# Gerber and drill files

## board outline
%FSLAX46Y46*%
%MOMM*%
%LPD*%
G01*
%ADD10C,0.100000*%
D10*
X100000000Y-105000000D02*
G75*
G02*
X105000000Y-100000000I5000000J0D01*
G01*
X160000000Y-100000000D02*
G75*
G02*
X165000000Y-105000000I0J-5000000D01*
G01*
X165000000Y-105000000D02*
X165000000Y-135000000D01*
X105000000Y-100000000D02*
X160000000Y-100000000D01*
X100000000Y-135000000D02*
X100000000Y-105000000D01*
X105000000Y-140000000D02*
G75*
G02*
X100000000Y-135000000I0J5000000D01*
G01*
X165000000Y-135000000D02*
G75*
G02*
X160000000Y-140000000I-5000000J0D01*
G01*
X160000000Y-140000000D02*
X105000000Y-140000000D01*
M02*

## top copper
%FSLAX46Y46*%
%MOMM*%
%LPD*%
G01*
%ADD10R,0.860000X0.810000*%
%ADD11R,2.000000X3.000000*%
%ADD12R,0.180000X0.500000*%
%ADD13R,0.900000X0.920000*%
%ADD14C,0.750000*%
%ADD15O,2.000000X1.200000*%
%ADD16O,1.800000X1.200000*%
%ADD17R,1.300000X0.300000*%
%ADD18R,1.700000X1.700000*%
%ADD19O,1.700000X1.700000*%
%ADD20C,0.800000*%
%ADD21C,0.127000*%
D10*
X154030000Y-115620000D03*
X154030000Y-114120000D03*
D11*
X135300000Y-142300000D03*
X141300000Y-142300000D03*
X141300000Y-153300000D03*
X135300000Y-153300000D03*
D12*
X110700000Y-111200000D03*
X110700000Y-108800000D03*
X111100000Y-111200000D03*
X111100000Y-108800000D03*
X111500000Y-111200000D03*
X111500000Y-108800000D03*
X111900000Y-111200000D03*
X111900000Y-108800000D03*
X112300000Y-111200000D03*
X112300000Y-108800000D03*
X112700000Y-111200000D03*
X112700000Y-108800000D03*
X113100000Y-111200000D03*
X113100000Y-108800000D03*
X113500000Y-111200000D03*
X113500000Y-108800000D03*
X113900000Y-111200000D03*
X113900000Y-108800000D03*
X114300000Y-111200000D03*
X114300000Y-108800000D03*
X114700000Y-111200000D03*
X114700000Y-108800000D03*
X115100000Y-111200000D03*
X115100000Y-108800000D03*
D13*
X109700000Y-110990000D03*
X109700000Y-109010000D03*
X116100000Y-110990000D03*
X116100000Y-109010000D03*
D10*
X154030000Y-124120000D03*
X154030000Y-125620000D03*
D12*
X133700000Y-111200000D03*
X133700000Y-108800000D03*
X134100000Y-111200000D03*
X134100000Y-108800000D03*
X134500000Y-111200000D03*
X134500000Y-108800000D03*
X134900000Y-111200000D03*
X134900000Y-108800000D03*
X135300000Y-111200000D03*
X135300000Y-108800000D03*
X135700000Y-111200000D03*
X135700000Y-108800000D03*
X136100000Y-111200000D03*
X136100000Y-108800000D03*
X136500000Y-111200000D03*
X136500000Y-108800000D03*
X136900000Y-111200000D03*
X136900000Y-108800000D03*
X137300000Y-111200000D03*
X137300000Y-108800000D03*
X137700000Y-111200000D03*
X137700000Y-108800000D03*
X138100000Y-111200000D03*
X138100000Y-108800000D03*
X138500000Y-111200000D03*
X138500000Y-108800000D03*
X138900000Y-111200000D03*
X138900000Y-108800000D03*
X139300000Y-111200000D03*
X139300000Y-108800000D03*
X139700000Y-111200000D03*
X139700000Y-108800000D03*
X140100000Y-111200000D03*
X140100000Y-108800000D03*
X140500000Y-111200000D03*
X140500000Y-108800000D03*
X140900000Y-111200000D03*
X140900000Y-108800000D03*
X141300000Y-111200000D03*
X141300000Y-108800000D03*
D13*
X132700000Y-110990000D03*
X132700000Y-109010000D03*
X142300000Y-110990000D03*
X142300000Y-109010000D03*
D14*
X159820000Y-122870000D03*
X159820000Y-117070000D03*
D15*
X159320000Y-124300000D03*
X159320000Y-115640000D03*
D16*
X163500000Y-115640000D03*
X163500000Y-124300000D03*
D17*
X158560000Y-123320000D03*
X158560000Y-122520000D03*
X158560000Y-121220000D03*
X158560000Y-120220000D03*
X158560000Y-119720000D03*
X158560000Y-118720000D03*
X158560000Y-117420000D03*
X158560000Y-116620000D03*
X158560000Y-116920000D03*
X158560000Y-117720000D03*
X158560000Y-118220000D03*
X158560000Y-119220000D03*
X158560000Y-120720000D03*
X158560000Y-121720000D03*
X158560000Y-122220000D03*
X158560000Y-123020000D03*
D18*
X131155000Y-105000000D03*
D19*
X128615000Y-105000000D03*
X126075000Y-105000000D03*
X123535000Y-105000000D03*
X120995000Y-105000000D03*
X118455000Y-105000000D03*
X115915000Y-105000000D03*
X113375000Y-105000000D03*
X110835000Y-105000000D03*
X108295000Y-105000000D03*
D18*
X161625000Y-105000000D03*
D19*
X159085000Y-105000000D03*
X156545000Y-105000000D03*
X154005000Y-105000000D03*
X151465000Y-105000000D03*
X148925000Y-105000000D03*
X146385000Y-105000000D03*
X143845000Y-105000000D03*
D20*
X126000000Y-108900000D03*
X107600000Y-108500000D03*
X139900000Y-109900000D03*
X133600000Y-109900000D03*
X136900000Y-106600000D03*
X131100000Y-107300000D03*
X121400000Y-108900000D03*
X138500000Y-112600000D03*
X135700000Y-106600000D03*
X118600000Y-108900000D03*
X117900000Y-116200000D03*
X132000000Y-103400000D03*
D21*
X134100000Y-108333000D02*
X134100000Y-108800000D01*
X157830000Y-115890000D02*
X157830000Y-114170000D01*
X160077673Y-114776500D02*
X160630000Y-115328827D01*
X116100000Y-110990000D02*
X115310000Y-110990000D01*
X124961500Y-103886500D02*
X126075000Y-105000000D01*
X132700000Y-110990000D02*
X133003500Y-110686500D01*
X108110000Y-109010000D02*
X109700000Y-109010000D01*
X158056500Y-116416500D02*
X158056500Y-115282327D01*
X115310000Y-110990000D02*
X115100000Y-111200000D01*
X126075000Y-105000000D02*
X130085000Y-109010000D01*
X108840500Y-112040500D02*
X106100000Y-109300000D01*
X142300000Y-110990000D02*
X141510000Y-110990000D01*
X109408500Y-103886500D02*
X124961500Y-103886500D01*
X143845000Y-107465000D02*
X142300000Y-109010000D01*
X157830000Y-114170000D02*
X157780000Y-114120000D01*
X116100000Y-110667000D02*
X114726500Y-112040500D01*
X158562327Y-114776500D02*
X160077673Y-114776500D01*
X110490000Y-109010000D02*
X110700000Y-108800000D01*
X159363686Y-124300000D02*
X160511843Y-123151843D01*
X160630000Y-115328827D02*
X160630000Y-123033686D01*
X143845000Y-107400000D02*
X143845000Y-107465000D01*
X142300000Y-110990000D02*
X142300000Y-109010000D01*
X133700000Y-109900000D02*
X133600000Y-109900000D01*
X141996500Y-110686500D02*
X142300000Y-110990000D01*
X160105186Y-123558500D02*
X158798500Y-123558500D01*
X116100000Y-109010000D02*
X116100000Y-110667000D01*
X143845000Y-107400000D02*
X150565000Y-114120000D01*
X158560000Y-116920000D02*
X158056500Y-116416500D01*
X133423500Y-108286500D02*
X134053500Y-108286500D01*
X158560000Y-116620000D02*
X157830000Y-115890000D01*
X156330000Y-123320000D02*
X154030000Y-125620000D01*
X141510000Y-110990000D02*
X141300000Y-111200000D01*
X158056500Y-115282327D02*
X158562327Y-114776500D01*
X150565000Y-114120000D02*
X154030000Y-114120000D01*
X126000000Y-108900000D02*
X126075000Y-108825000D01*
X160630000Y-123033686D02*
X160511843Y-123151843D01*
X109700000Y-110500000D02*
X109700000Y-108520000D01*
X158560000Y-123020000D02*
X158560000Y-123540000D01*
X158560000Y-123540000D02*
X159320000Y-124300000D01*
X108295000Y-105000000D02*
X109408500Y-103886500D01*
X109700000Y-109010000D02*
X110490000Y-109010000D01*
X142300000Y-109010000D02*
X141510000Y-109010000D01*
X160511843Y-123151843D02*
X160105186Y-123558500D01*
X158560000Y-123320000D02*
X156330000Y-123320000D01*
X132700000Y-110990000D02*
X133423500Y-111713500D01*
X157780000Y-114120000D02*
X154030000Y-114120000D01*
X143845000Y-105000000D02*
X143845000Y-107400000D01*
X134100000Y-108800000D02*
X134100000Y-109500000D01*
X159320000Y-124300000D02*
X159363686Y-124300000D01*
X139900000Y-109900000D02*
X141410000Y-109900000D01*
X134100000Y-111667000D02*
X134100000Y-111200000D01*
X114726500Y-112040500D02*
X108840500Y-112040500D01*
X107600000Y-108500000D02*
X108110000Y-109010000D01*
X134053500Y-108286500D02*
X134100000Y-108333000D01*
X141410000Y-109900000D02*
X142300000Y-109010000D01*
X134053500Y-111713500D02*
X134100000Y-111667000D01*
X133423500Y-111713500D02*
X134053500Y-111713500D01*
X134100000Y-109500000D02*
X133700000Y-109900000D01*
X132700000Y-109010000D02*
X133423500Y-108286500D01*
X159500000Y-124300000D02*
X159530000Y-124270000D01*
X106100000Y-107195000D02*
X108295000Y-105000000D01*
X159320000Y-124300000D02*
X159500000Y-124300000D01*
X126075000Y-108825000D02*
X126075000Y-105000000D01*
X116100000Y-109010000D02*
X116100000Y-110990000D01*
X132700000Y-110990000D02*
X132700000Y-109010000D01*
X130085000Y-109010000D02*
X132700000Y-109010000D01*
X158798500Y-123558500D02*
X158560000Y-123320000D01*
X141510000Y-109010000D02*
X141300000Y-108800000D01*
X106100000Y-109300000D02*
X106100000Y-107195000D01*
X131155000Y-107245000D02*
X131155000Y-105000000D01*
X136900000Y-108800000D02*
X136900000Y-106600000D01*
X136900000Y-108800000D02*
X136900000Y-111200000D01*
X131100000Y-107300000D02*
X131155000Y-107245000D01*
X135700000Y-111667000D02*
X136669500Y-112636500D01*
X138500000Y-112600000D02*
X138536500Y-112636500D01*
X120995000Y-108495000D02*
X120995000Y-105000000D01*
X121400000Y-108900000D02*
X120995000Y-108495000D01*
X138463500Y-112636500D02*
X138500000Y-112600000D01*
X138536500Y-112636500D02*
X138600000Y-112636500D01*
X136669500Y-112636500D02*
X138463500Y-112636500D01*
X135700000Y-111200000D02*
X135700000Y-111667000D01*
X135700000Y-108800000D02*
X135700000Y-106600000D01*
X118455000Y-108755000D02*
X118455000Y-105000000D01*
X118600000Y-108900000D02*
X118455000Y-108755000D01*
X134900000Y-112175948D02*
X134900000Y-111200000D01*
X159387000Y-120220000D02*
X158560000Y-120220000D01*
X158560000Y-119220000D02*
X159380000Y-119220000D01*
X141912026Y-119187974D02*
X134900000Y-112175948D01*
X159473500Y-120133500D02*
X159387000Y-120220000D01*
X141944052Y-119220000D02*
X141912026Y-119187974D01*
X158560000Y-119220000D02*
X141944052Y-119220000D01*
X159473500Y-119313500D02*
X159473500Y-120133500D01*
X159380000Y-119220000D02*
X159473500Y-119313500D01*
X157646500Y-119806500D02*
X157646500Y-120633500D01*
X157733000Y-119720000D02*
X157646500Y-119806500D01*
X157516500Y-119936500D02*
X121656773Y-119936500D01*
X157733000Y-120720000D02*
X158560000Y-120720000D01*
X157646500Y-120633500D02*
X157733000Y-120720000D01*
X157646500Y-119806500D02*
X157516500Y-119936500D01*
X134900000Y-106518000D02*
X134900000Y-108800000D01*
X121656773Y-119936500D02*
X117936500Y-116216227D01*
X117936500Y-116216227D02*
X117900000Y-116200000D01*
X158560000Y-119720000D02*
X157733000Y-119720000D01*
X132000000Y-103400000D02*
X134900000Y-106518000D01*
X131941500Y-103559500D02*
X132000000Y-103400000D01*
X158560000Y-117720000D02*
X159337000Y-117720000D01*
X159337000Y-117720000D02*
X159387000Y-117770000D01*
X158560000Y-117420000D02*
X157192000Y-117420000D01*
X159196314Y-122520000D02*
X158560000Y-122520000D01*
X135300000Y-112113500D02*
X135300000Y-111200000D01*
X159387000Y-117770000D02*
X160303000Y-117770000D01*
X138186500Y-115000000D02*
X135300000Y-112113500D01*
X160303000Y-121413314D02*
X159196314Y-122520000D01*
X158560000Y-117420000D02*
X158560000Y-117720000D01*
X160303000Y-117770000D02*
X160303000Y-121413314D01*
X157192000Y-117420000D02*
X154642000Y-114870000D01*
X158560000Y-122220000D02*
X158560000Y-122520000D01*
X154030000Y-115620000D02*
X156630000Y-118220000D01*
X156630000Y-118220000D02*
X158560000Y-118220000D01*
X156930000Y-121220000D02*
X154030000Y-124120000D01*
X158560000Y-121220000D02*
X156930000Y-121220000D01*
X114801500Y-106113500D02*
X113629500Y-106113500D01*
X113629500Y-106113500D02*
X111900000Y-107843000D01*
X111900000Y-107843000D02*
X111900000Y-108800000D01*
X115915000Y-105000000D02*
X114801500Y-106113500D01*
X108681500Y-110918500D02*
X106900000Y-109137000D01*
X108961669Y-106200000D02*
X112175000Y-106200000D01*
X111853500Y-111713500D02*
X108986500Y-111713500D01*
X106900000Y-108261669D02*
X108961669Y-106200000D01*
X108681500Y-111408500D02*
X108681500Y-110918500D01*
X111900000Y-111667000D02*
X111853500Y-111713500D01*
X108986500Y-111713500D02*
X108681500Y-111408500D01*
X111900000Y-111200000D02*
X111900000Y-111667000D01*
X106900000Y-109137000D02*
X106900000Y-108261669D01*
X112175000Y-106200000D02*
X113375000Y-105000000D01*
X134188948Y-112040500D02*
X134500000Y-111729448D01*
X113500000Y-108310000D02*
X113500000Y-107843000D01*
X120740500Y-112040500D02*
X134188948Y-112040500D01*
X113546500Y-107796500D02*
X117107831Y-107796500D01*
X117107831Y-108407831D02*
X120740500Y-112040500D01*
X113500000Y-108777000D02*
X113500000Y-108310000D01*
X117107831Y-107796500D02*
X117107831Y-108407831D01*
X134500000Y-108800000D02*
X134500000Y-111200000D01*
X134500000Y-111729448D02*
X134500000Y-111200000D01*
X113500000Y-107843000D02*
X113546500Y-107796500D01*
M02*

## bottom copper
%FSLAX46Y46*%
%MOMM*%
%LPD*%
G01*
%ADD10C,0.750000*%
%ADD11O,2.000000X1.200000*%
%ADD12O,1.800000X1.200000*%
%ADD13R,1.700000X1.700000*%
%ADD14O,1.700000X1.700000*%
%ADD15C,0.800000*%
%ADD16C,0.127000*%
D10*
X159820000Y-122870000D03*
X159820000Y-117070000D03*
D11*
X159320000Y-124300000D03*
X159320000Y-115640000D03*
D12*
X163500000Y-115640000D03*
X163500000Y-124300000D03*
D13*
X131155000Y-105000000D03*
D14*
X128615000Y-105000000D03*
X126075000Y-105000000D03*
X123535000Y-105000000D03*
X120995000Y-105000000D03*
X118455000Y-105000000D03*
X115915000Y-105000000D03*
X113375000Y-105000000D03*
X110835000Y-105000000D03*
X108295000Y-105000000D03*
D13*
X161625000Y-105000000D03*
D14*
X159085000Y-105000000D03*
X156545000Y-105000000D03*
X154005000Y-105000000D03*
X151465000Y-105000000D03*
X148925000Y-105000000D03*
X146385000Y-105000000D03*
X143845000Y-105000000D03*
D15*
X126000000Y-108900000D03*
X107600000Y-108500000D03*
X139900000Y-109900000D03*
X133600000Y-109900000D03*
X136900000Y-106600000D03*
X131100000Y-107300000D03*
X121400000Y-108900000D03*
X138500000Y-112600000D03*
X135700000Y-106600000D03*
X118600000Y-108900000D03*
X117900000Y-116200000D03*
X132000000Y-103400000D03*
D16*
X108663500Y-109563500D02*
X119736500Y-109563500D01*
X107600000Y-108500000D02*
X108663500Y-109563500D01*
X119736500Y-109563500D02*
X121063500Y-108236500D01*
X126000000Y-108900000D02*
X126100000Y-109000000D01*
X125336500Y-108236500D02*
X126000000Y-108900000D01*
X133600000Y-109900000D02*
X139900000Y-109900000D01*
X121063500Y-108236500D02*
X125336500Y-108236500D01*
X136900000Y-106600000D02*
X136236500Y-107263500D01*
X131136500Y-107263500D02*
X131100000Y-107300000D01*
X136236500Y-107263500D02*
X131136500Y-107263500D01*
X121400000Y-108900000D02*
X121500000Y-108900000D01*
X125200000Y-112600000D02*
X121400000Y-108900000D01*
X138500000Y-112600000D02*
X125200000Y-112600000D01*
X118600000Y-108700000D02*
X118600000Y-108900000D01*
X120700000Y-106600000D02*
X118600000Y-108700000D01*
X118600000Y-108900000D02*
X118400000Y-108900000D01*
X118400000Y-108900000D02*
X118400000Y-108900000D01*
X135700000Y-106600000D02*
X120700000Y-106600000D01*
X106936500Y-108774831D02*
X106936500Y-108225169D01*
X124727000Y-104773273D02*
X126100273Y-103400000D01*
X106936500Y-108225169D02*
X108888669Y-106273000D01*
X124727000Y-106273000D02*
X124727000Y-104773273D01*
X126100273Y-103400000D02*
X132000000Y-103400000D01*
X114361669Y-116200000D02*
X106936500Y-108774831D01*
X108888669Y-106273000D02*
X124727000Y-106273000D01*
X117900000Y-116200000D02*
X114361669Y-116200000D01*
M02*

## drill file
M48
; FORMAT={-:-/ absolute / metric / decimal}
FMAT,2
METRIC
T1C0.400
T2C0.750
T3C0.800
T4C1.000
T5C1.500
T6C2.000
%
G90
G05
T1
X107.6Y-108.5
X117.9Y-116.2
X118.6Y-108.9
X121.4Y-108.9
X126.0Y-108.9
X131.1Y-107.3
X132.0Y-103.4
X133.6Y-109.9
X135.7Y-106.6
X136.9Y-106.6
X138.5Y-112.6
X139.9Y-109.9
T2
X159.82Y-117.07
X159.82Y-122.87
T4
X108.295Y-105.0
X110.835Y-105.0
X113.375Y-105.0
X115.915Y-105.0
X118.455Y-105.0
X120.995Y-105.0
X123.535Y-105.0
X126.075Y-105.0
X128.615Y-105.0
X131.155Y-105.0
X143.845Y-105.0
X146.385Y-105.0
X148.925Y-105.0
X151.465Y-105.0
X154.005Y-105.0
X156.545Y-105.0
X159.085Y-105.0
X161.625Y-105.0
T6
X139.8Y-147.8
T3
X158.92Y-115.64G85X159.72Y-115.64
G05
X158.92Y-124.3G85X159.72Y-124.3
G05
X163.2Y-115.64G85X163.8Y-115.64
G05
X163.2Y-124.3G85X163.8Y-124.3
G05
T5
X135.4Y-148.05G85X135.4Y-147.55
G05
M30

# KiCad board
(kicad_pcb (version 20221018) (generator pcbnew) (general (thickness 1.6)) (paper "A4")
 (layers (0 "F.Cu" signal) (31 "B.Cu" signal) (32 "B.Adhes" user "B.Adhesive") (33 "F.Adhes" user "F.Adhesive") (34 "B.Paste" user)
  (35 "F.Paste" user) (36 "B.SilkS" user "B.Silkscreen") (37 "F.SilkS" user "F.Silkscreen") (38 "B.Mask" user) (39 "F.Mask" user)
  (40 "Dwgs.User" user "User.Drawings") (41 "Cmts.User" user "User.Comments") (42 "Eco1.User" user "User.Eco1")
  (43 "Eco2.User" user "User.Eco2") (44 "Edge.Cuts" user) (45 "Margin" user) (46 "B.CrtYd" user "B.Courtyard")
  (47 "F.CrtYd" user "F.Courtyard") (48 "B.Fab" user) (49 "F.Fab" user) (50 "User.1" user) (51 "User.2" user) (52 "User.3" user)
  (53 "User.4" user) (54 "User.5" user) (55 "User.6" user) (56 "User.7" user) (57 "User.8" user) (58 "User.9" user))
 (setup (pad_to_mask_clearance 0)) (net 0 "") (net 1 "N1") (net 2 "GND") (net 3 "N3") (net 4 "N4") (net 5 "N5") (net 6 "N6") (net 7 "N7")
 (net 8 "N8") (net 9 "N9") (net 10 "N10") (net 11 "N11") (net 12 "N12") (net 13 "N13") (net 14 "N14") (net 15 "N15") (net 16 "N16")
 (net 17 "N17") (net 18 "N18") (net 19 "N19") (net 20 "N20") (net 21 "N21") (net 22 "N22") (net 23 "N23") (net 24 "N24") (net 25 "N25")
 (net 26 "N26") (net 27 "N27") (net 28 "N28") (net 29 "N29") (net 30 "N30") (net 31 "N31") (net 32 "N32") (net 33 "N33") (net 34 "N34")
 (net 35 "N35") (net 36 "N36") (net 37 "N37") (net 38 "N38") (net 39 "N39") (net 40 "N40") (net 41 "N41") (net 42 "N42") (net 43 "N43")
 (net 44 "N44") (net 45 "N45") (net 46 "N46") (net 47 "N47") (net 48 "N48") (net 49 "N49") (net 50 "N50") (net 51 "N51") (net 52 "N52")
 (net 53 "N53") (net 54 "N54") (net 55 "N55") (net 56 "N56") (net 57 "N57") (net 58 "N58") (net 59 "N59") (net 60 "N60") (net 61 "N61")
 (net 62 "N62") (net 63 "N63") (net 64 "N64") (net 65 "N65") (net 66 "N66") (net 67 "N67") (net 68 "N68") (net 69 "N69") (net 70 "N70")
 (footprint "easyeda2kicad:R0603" (layer "F.Cu") (at 154.03 114.87 90)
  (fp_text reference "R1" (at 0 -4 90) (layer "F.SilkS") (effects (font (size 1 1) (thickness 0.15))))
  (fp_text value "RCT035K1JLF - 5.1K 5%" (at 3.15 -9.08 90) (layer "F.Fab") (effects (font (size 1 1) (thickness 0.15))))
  (pad "1" smd rect (at -0.75 0 90) (size 0.81 0.86) (layers "F.Cu" "F.Paste" "F.Mask") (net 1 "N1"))
  (pad "2" smd rect (at 0.75 0 90) (size 0.81 0.86) (layers "F.Cu" "F.Paste" "F.Mask") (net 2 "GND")))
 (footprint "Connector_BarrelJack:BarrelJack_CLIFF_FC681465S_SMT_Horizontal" (layer "F.Cu") (at 138.3 147.8)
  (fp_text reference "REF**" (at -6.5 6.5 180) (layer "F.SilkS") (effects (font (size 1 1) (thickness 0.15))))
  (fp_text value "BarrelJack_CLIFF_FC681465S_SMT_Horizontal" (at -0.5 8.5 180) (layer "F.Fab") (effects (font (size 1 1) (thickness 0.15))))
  (pad "" np_thru_hole oval (at -2.9 0 90) (size 2 1.5) (drill oval 2 1.5) (layers "*.Cu" "*.Mask"))
  (pad "" np_thru_hole circle (at 1.5 0 90) (size 2 2) (drill 2) (layers "*.Cu" "*.Mask"))
  (pad "1" smd rect (at -3 -5.5 90) (size 3 2) (layers "F.Cu" "F.Paste" "F.Mask"))
  (pad "1" smd rect (at 3 -5.5 90) (size 3 2) (layers "F.Cu" "F.Paste" "F.Mask"))
  (pad "2" smd rect (at 3 5.5 90) (size 3 2) (layers "F.Cu" "F.Paste" "F.Mask"))
  (pad "3" smd rect (at -3 5.5 90) (size 3 2) (layers "F.Cu" "F.Paste" "F.Mask")))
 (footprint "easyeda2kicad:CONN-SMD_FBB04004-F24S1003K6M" (layer "F.Cu") (at 112.9 110)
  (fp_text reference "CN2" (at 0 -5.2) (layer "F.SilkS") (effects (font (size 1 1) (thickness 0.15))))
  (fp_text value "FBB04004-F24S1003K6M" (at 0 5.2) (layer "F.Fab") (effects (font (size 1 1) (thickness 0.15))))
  (pad "1" smd rect (at -2.2 1.2) (size 0.18 0.5) (layers "F.Cu" "F.Paste" "F.Mask") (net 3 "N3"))
  (pad "2" smd rect (at -2.2 -1.2) (size 0.18 0.5) (layers "F.Cu" "F.Paste" "F.Mask") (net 2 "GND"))
  (pad "3" smd rect (at -1.8 1.2) (size 0.18 0.5) (layers "F.Cu" "F.Paste" "F.Mask") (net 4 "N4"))
  (pad "4" smd rect (at -1.8 -1.2) (size 0.18 0.5) (layers "F.Cu" "F.Paste" "F.Mask") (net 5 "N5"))
  (pad "5" smd rect (at -1.4 1.2) (size 0.18 0.5) (layers "F.Cu" "F.Paste" "F.Mask") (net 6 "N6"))
  (pad "6" smd rect (at -1.4 -1.2) (size 0.18 0.5) (layers "F.Cu" "F.Paste" "F.Mask") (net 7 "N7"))
  (pad "7" smd rect (at -1 1.2) (size 0.18 0.5) (layers "F.Cu" "F.Paste" "F.Mask") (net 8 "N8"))
  (pad "8" smd rect (at -1 -1.2) (size 0.18 0.5) (layers "F.Cu" "F.Paste" "F.Mask") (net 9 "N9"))
  (pad "9" smd rect (at -0.6 1.2) (size 0.18 0.5) (layers "F.Cu" "F.Paste" "F.Mask") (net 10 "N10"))
  (pad "10" smd rect (at -0.6 -1.2) (size 0.18 0.5) (layers "F.Cu" "F.Paste" "F.Mask") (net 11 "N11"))
  (pad "11" smd rect (at -0.2 1.2) (size 0.18 0.5) (layers "F.Cu" "F.Paste" "F.Mask") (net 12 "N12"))
  (pad "12" smd rect (at -0.2 -1.2) (size 0.18 0.5) (layers "F.Cu" "F.Paste" "F.Mask") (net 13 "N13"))
  (pad "13" smd rect (at 0.2 1.2) (size 0.18 0.5) (layers "F.Cu" "F.Paste" "F.Mask") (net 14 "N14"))
  (pad "14" smd rect (at 0.2 -1.2) (size 0.18 0.5) (layers "F.Cu" "F.Paste" "F.Mask") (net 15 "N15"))
  (pad "15" smd rect (at 0.6 1.2) (size 0.18 0.5) (layers "F.Cu" "F.Paste" "F.Mask") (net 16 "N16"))
  (pad "16" smd rect (at 0.6 -1.2) (size 0.18 0.5) (layers "F.Cu" "F.Paste" "F.Mask") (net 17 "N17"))
  (pad "17" smd rect (at 1 1.2) (size 0.18 0.5) (layers "F.Cu" "F.Paste" "F.Mask") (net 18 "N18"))
  (pad "18" smd rect (at 1 -1.2) (size 0.18 0.5) (layers "F.Cu" "F.Paste" "F.Mask") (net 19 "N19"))
  (pad "19" smd rect (at 1.4 1.2) (size 0.18 0.5) (layers "F.Cu" "F.Paste" "F.Mask") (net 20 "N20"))
  (pad "20" smd rect (at 1.4 -1.2) (size 0.18 0.5) (layers "F.Cu" "F.Paste" "F.Mask") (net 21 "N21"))
  (pad "21" smd rect (at 1.8 1.2) (size 0.18 0.5) (layers "F.Cu" "F.Paste" "F.Mask") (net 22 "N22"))
  (pad "22" smd rect (at 1.8 -1.2) (size 0.18 0.5) (layers "F.Cu" "F.Paste" "F.Mask") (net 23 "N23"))
  (pad "23" smd rect (at 2.2 1.2) (size 0.18 0.5) (layers "F.Cu" "F.Paste" "F.Mask") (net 2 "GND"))
  (pad "24" smd rect (at 2.2 -1.2) (size 0.18 0.5) (layers "F.Cu" "F.Paste" "F.Mask") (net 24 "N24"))
  (pad "25" smd rect (at -3.2 0.99) (size 0.9 0.92) (layers "F.Cu" "F.Paste" "F.Mask") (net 2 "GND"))
  (pad "26" smd rect (at -3.2 -0.99) (size 0.9 0.92) (layers "F.Cu" "F.Paste" "F.Mask") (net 2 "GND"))
  (pad "27" smd rect (at 3.2 0.99) (size 0.9 0.92) (layers "F.Cu" "F.Paste" "F.Mask") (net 2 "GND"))
  (pad "28" smd rect (at 3.2 -0.99) (size 0.9 0.92) (layers "F.Cu" "F.Paste" "F.Mask") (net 2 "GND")))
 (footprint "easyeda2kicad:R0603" (layer "F.Cu") (at 154.03 124.87 -90)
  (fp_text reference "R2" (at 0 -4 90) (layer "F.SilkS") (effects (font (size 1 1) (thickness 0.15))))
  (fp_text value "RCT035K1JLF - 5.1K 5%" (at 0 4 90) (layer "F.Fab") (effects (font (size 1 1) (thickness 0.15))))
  (pad "1" smd rect (at -0.75 0 270) (size 0.81 0.86) (layers "F.Cu" "F.Paste" "F.Mask") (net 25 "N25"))
  (pad "2" smd rect (at 0.75 0 270) (size 0.81 0.86) (layers "F.Cu" "F.Paste" "F.Mask") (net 2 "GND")))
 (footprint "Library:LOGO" (layer "F.Cu") (at 156.4 132.7)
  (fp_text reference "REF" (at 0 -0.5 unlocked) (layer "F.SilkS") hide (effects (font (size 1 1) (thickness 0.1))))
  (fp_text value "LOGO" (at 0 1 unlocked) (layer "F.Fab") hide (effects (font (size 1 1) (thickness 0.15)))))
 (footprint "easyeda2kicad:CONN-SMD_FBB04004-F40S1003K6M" (layer "F.Cu") (at 137.5 110)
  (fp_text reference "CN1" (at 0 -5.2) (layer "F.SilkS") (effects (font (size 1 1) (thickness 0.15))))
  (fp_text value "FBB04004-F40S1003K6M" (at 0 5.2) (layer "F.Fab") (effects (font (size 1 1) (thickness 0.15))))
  (pad "1" smd rect (at -3.8 1.2) (size 0.18 0.5) (layers "F.Cu" "F.Paste" "F.Mask") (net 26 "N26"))
  (pad "2" smd rect (at -3.8 -1.2) (size 0.18 0.5) (layers "F.Cu" "F.Paste" "F.Mask") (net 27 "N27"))
  (pad "3" smd rect (at -3.4 1.2) (size 0.18 0.5) (layers "F.Cu" "F.Paste" "F.Mask") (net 2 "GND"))
  (pad "4" smd rect (at -3.4 -1.2) (size 0.18 0.5) (layers "F.Cu" "F.Paste" "F.Mask") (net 2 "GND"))
  (pad "5" smd rect (at -3 1.2) (size 0.18 0.5) (layers "F.Cu" "F.Paste" "F.Mask") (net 17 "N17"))
  (pad "6" smd rect (at -3 -1.2) (size 0.18 0.5) (layers "F.Cu" "F.Paste" "F.Mask") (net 17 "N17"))
  (pad "7" smd rect (at -2.6 1.2) (size 0.18 0.5) (layers "F.Cu" "F.Paste" "F.Mask") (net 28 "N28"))
  (pad "8" smd rect (at -2.6 -1.2) (size 0.18 0.5) (layers "F.Cu" "F.Paste" "F.Mask") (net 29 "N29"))
  (pad "9" smd rect (at -2.2 1.2) (size 0.18 0.5) (layers "F.Cu" "F.Paste" "F.Mask") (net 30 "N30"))
  (pad "10" smd rect (at -2.2 -1.2) (size 0.18 0.5) (layers "F.Cu" "F.Paste" "F.Mask") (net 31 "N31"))
  (pad "11" smd rect (at -1.8 1.2) (size 0.18 0.5) (layers "F.Cu" "F.Paste" "F.Mask") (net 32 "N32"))
  (pad "12" smd rect (at -1.8 -1.2) (size 0.18 0.5) (layers "F.Cu" "F.Paste" "F.Mask") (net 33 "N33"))
  (pad "13" smd rect (at -1.4 1.2) (size 0.18 0.5) (layers "F.Cu" "F.Paste" "F.Mask") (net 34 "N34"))
  (pad "14" smd rect (at -1.4 -1.2) (size 0.18 0.5) (layers "F.Cu" "F.Paste" "F.Mask") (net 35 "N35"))
  (pad "15" smd rect (at -1 1.2) (size 0.18 0.5) (layers "F.Cu" "F.Paste" "F.Mask") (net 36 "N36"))
  (pad "16" smd rect (at -1 -1.2) (size 0.18 0.5) (layers "F.Cu" "F.Paste" "F.Mask") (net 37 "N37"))
  (pad "17" smd rect (at -0.6 1.2) (size 0.18 0.5) (layers "F.Cu" "F.Paste" "F.Mask") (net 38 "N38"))
  (pad "18" smd rect (at -0.6 -1.2) (size 0.18 0.5) (layers "F.Cu" "F.Paste" "F.Mask") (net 38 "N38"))
  (pad "19" smd rect (at -0.2 1.2) (size 0.18 0.5) (layers "F.Cu" "F.Paste" "F.Mask") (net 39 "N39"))
  (pad "20" smd rect (at -0.2 -1.2) (size 0.18 0.5) (layers "F.Cu" "F.Paste" "F.Mask") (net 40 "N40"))
  (pad "21" smd rect (at 0.2 1.2) (size 0.18 0.5) (layers "F.Cu" "F.Paste" "F.Mask") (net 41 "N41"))
  (pad "22" smd rect (at 0.2 -1.2) (size 0.18 0.5) (layers "F.Cu" "F.Paste" "F.Mask") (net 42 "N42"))
  (pad "23" smd rect (at 0.6 1.2) (size 0.18 0.5) (layers "F.Cu" "F.Paste" "F.Mask") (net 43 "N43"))
  (pad "24" smd rect (at 0.6 -1.2) (size 0.18 0.5) (layers "F.Cu" "F.Paste" "F.Mask") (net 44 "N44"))
  (pad "25" smd rect (at 1 1.2) (size 0.18 0.5) (layers "F.Cu" "F.Paste" "F.Mask") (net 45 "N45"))
  (pad "26" smd rect (at 1 -1.2) (size 0.18 0.5) (layers "F.Cu" "F.Paste" "F.Mask") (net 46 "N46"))
  (pad "27" smd rect (at 1.4 1.2) (size 0.18 0.5) (layers "F.Cu" "F.Paste" "F.Mask") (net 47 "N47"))
  (pad "28" smd rect (at 1.4 -1.2) (size 0.18 0.5) (layers "F.Cu" "F.Paste" "F.Mask") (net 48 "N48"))
  (pad "29" smd rect (at 1.8 1.2) (size 0.18 0.5) (layers "F.Cu" "F.Paste" "F.Mask") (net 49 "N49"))
  (pad "30" smd rect (at 1.8 -1.2) (size 0.18 0.5) (layers "F.Cu" "F.Paste" "F.Mask") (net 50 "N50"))
  (pad "31" smd rect (at 2.2 1.2) (size 0.18 0.5) (layers "F.Cu" "F.Paste" "F.Mask") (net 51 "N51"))
  (pad "32" smd rect (at 2.2 -1.2) (size 0.18 0.5) (layers "F.Cu" "F.Paste" "F.Mask") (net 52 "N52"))
  (pad "33" smd rect (at 2.6 1.2) (size 0.18 0.5) (layers "F.Cu" "F.Paste" "F.Mask") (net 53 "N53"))
  (pad "34" smd rect (at 2.6 -1.2) (size 0.18 0.5) (layers "F.Cu" "F.Paste" "F.Mask") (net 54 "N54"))
  (pad "35" smd rect (at 3 1.2) (size 0.18 0.5) (layers "F.Cu" "F.Paste" "F.Mask") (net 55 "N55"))
  (pad "36" smd rect (at 3 -1.2) (size 0.18 0.5) (layers "F.Cu" "F.Paste" "F.Mask") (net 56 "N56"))
  (pad "37" smd rect (at 3.4 1.2) (size 0.18 0.5) (layers "F.Cu" "F.Paste" "F.Mask") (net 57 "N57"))
  (pad "38" smd rect (at 3.4 -1.2) (size 0.18 0.5) (layers "F.Cu" "F.Paste" "F.Mask") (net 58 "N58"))
  (pad "39" smd rect (at 3.8 1.2) (size 0.18 0.5) (layers "F.Cu" "F.Paste" "F.Mask") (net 2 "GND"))
  (pad "40" smd rect (at 3.8 -1.2) (size 0.18 0.5) (layers "F.Cu" "F.Paste" "F.Mask") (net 2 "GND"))
  (pad "41" smd rect (at -4.8 0.99) (size 0.9 0.92) (layers "F.Cu" "F.Paste" "F.Mask") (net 2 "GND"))
  (pad "42" smd rect (at -4.8 -0.99) (size 0.9 0.92) (layers "F.Cu" "F.Paste" "F.Mask") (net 2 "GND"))
  (pad "43" smd rect (at 4.8 0.99) (size 0.9 0.92) (layers "F.Cu" "F.Paste" "F.Mask") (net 2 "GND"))
  (pad "44" smd rect (at 4.8 -0.99) (size 0.9 0.92) (layers "F.Cu" "F.Paste" "F.Mask") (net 2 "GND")))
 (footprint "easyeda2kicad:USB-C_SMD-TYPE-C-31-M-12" (layer "F.Cu") (at 161.03 119.97 90)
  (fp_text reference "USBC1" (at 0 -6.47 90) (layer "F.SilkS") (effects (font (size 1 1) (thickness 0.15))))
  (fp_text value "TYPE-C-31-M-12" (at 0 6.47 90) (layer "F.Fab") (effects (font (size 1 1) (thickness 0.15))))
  (pad "" thru_hole circle (at -2.9 -1.21 90) (size 0.75 0.75) (drill 0.75) (layers "*.Cu" "*.Mask"))
  (pad "" thru_hole circle (at 2.9 -1.21 90) (size 0.75 0.75) (drill 0.75) (layers "*.Cu" "*.Mask"))
  (pad "0" thru_hole oval (at -4.33 -1.71 90) (size 1.2 2) (drill oval 0.799998 1.600022) (layers "*.Cu" "*.Mask") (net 2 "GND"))
  (pad "1" thru_hole oval (at 4.33 -1.71 90) (size 1.2 2) (drill oval 0.799998 1.599971) (layers "*.Cu" "*.Mask"))
  (pad "2" thru_hole oval (at 4.33 2.47 90) (size 1.2 1.8) (drill oval 0.799998 1.399997) (layers "*.Cu" "*.Mask"))
  (pad "3" thru_hole oval (at -4.33 2.47 90) (size 1.2 1.8) (drill oval 0.799998 1.399997) (layers "*.Cu" "*.Mask"))
  (pad "A1" smd rect (at -3.35 -2.47 90) (size 0.3 1.3) (layers "F.Cu" "F.Paste" "F.Mask") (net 2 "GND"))
  (pad "A4" smd rect (at -2.55 -2.47 90) (size 0.3 1.3) (layers "F.Cu" "F.Paste" "F.Mask") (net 30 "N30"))
  (pad "A5" smd rect (at -1.25 -2.47 90) (size 0.3 1.3) (layers "F.Cu" "F.Paste" "F.Mask") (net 25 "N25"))
  (pad "A6" smd rect (at -0.25 -2.47 90) (size 0.3 1.3) (layers "F.Cu" "F.Paste" "F.Mask") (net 28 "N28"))
  (pad "A7" smd rect (at 0.25 -2.47 90) (size 0.3 1.3) (layers "F.Cu" "F.Paste" "F.Mask") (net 29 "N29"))
  (pad "A8" smd rect (at 1.25 -2.47 90) (size 0.3 1.3) (layers "F.Cu" "F.Paste" "F.Mask") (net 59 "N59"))
  (pad "A9" smd rect (at 2.55 -2.47 90) (size 0.3 1.3) (layers "F.Cu" "F.Paste" "F.Mask") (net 30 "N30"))
  (pad "A12" smd rect (at 3.35 -2.47 90) (size 0.3 1.3) (layers "F.Cu" "F.Paste" "F.Mask") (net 2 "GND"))
  (pad "B1" smd rect (at 3.05 -2.47 90) (size 0.3 1.3) (layers "F.Cu" "F.Paste" "F.Mask") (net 2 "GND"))
  (pad "B4" smd rect (at 2.25 -2.47 90) (size 0.3 1.3) (layers "F.Cu" "F.Paste" "F.Mask") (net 30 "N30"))
  (pad "B5" smd rect (at 1.75 -2.47 90) (size 0.3 1.3) (layers "F.Cu" "F.Paste" "F.Mask") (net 1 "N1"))
  (pad "B6" smd rect (at 0.75 -2.47 90) (size 0.3 1.3) (layers "F.Cu" "F.Paste" "F.Mask") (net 28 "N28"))
  (pad "B7" smd rect (at -0.75 -2.47 90) (size 0.3 1.3) (layers "F.Cu" "F.Paste" "F.Mask") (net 29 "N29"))
  (pad "B8" smd rect (at -1.75 -2.47 90) (size 0.3 1.3) (layers "F.Cu" "F.Paste" "F.Mask") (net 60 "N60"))
  (pad "B9" smd rect (at -2.25 -2.47 90) (size 0.3 1.3) (layers "F.Cu" "F.Paste" "F.Mask") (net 30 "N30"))
  (pad "B12" smd rect (at -3.05 -2.47 90) (size 0.3 1.3) (layers "F.Cu" "F.Paste" "F.Mask") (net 2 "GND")))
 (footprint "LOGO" (layer "B.Cu") (at 156.4 132.7 180)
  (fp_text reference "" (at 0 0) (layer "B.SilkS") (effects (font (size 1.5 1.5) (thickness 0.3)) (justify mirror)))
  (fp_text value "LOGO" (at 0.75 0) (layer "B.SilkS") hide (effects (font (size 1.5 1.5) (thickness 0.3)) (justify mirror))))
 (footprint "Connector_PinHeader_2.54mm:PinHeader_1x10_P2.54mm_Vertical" (layer "B.Cu") (at 131.155 105 90)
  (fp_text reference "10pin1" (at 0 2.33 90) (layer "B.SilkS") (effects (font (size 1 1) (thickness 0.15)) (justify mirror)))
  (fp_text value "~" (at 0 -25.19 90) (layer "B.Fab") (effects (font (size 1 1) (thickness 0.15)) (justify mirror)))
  (pad "1" thru_hole rect (at 0 0 90) (size 1.7 1.7) (drill 1) (layers "*.Cu" "*.Mask") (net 38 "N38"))
  (pad "2" thru_hole oval (at 0 -2.54 90) (size 1.7 1.7) (drill 1) (layers "*.Cu" "*.Mask") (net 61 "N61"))
  (pad "3" thru_hole oval (at 0 -5.08 90) (size 1.7 1.7) (drill 1) (layers "*.Cu" "*.Mask") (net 2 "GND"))
  (pad "4" thru_hole oval (at 0 -7.62 90) (size 1.7 1.7) (drill 1) (layers "*.Cu" "*.Mask") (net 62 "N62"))
  (pad "5" thru_hole oval (at 0 -10.16 90) (size 1.7 1.7) (drill 1) (layers "*.Cu" "*.Mask") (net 32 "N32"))
  (pad "6" thru_hole oval (at 0 -12.7 90) (size 1.7 1.7) (drill 1) (layers "*.Cu" "*.Mask") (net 33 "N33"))
  (pad "7" thru_hole oval (at 0 -15.24 90) (size 1.7 1.7) (drill 1) (layers "*.Cu" "*.Mask") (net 9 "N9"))
  (pad "8" thru_hole oval (at 0 -17.78 90) (size 1.7 1.7) (drill 1) (layers "*.Cu" "*.Mask") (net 8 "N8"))
  (pad "9" thru_hole oval (at 0 -20.32 90) (size 1.7 1.7) (drill 1) (layers "*.Cu" "*.Mask") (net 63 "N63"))
  (pad "10" thru_hole oval (at 0 -22.86 90) (size 1.7 1.7) (drill 1) (layers "*.Cu" "*.Mask") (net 2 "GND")))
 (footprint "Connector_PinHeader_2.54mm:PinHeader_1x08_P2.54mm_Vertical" (layer "B.Cu") (at 161.625 105 90)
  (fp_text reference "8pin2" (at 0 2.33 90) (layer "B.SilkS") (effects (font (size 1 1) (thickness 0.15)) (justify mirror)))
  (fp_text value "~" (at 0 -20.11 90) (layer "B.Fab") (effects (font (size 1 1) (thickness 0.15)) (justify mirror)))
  (pad "1" thru_hole rect (at 0 0 90) (size 1.7 1.7) (drill 1) (layers "*.Cu" "*.Mask") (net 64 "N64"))
  (pad "2" thru_hole oval (at 0 -2.54 90) (size 1.7 1.7) (drill 1) (layers "*.Cu" "*.Mask") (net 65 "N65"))
  (pad "3" thru_hole oval (at 0 -5.08 90) (size 1.7 1.7) (drill 1) (layers "*.Cu" "*.Mask") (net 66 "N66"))
  (pad "4" thru_hole oval (at 0 -7.62 90) (size 1.7 1.7) (drill 1) (layers "*.Cu" "*.Mask") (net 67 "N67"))
  (pad "5" thru_hole oval (at 0 -10.16 90) (size 1.7 1.7) (drill 1) (layers "*.Cu" "*.Mask") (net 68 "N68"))
  (pad "6" thru_hole oval (at 0 -12.7 90) (size 1.7 1.7) (drill 1) (layers "*.Cu" "*.Mask") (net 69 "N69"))
  (pad "7" thru_hole oval (at 0 -15.24 90) (size 1.7 1.7) (drill 1) (layers "*.Cu" "*.Mask") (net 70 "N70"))
  (pad "8" thru_hole oval (at 0 -17.78 90) (size 1.7 1.7) (drill 1) (layers "*.Cu" "*.Mask") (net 2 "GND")))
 (gr_arc (start 100 105) (mid 101.464466 101.464466) (end 105 100) (stroke (width 0.1) (type default)) (layer "Edge.Cuts"))
 (gr_arc (start 160 100) (mid 163.535533 101.464466) (end 165 105) (stroke (width 0.1) (type default)) (layer "Edge.Cuts"))
 (gr_line (start 165 105) (end 165 135) (stroke (width 0.1) (type default)) (layer "Edge.Cuts"))
 (gr_line (start 105 100) (end 160 100) (stroke (width 0.1) (type default)) (layer "Edge.Cuts"))
 (gr_line (start 100 135) (end 100 105) (stroke (width 0.1) (type default)) (layer "Edge.Cuts"))
 (gr_arc (start 105 140) (mid 101.464466 138.535534) (end 100 135) (stroke (width 0.1) (type default)) (layer "Edge.Cuts"))
 (gr_arc (start 165 135) (mid 163.535534 138.535533) (end 160 140) (stroke (width 0.1) (type default)) (layer "Edge.Cuts"))
 (gr_line (start 160 140) (end 105 140) (stroke (width 0.1) (type default)) (layer "Edge.Cuts"))
 (segment (start 134.1 108.333) (end 134.1 108.8) (width 0.127) (layer "F.Cu") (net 2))
 (segment (start 157.83 115.89) (end 157.83 114.17) (width 0.127) (layer "F.Cu") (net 2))
 (segment (start 160.077673 114.7765) (end 160.63 115.328827) (width 0.127) (layer "F.Cu") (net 2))
 (segment (start 116.1 110.99) (end 115.31 110.99) (width 0.127) (layer "F.Cu") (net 2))
 (segment (start 124.9615 103.8865) (end 126.075 105) (width 0.127) (layer "F.Cu") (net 2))
 (segment (start 132.7 110.99) (end 133.0035 110.6865) (width 0.127) (layer "F.Cu") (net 2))
 (segment (start 108.11 109.01) (end 109.7 109.01) (width 0.127) (layer "F.Cu") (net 2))
 (segment (start 158.0565 116.4165) (end 158.0565 115.282327) (width 0.127) (layer "F.Cu") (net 2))
 (segment (start 115.31 110.99) (end 115.1 111.2) (width 0.127) (layer "F.Cu") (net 2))
 (segment (start 126.075 105) (end 130.085 109.01) (width 0.127) (layer "F.Cu") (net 2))
 (segment (start 108.8405 112.0405) (end 106.1 109.3) (width 0.127) (layer "F.Cu") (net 2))
 (segment (start 142.3 110.99) (end 141.51 110.99) (width 0.127) (layer "F.Cu") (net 2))
 (segment (start 109.4085 103.8865) (end 124.9615 103.8865) (width 0.127) (layer "F.Cu") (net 2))
 (segment (start 143.845 107.465) (end 142.3 109.01) (width 0.127) (layer "F.Cu") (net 2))
 (segment (start 157.83 114.17) (end 157.78 114.12) (width 0.127) (layer "F.Cu") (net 2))
 (segment (start 116.1 110.667) (end 114.7265 112.0405) (width 0.127) (layer "F.Cu") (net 2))
 (segment (start 158.562327 114.7765) (end 160.077673 114.7765) (width 0.127) (layer "F.Cu") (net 2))
 (segment (start 110.49 109.01) (end 110.7 108.8) (width 0.127) (layer "F.Cu") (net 2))
 (segment (start 159.363686 124.3) (end 160.511843 123.151843) (width 0.127) (layer "F.Cu") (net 2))
 (segment (start 160.63 115.328827) (end 160.63 123.033686) (width 0.127) (layer "F.Cu") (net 2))
 (segment (start 143.845 107.4) (end 143.845 107.465) (width 0.127) (layer "F.Cu") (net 2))
 (segment (start 142.3 110.99) (end 142.3 109.01) (width 0.127) (layer "F.Cu") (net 2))
 (segment (start 133.7 109.9) (end 133.6 109.9) (width 0.127) (layer "F.Cu") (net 2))
 (segment (start 141.9965 110.6865) (end 142.3 110.99) (width 0.127) (layer "F.Cu") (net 2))
 (segment (start 160.105186 123.5585) (end 158.7985 123.5585) (width 0.127) (layer "F.Cu") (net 2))
 (segment (start 116.1 109.01) (end 116.1 110.667) (width 0.127) (layer "F.Cu") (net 2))
 (segment (start 143.845 107.4) (end 150.565 114.12) (width 0.127) (layer "F.Cu") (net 2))
 (segment (start 158.56 116.92) (end 158.0565 116.4165) (width 0.127) (layer "F.Cu") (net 2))
 (segment (start 133.4235 108.2865) (end 134.0535 108.2865) (width 0.127) (layer "F.Cu") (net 2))
 (segment (start 158.56 116.62) (end 157.83 115.89) (width 0.127) (layer "F.Cu") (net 2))
 (segment (start 156.33 123.32) (end 154.03 125.62) (width 0.127) (layer "F.Cu") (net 2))
 (segment (start 141.51 110.99) (end 141.3 111.2) (width 0.127) (layer "F.Cu") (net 2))
 (segment (start 158.0565 115.282327) (end 158.562327 114.7765) (width 0.127) (layer "F.Cu") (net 2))
 (segment (start 150.565 114.12) (end 154.03 114.12) (width 0.127) (layer "F.Cu") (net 2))
 (segment (start 126 108.9) (end 126.075 108.825) (width 0.127) (layer "F.Cu") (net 2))
 (segment (start 160.63 123.033686) (end 160.511843 123.151843) (width 0.127) (layer "F.Cu") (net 2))
 (segment (start 109.7 110.5) (end 109.7 108.52) (width 0.127) (layer "F.Cu") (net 2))
 (segment (start 158.56 123.02) (end 158.56 123.54) (width 0.127) (layer "F.Cu") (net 2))
 (segment (start 158.56 123.54) (end 159.32 124.3) (width 0.127) (layer "F.Cu") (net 2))
 (segment (start 108.295 105) (end 109.4085 103.8865) (width 0.127) (layer "F.Cu") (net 2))
 (segment (start 109.7 109.01) (end 110.49 109.01) (width 0.127) (layer "F.Cu") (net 2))
 (segment (start 142.3 109.01) (end 141.51 109.01) (width 0.127) (layer "F.Cu") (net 2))
 (segment (start 160.511843 123.151843) (end 160.105186 123.5585) (width 0.127) (layer "F.Cu") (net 2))
 (segment (start 158.56 123.32) (end 156.33 123.32) (width 0.127) (layer "F.Cu") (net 2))
 (segment (start 132.7 110.99) (end 133.4235 111.7135) (width 0.127) (layer "F.Cu") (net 2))
 (segment (start 157.78 114.12) (end 154.03 114.12) (width 0.127) (layer "F.Cu") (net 2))
 (segment (start 143.845 105) (end 143.845 107.4) (width 0.127) (layer "F.Cu") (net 2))
 (segment (start 134.1 108.8) (end 134.1 109.5) (width 0.127) (layer "F.Cu") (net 2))
 (segment (start 159.32 124.3) (end 159.363686 124.3) (width 0.127) (layer "F.Cu") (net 2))
 (segment (start 139.9 109.9) (end 141.41 109.9) (width 0.127) (layer "F.Cu") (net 2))
 (segment (start 134.1 111.667) (end 134.1 111.2) (width 0.127) (layer "F.Cu") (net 2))
 (segment (start 114.7265 112.0405) (end 108.8405 112.0405) (width 0.127) (layer "F.Cu") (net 2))
 (segment (start 107.6 108.5) (end 108.11 109.01) (width 0.127) (layer "F.Cu") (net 2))
 (segment (start 134.0535 108.2865) (end 134.1 108.333) (width 0.127) (layer "F.Cu") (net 2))
 (segment (start 141.41 109.9) (end 142.3 109.01) (width 0.127) (layer "F.Cu") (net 2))
 (segment (start 134.0535 111.7135) (end 134.1 111.667) (width 0.127) (layer "F.Cu") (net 2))
 (segment (start 133.4235 111.7135) (end 134.0535 111.7135) (width 0.127) (layer "F.Cu") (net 2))
 (segment (start 134.1 109.5) (end 133.7 109.9) (width 0.127) (layer "F.Cu") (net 2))
 (segment (start 132.7 109.01) (end 133.4235 108.2865) (width 0.127) (layer "F.Cu") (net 2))
 (segment (start 159.5 124.3) (end 159.53 124.27) (width 0.127) (layer "F.Cu") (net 2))
 (segment (start 106.1 107.195) (end 108.295 105) (width 0.127) (layer "F.Cu") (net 2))
 (segment (start 159.32 124.3) (end 159.5 124.3) (width 0.127) (layer "F.Cu") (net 2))
 (segment (start 126.075 108.825) (end 126.075 105) (width 0.127) (layer "F.Cu") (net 2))
 (segment (start 116.1 109.01) (end 116.1 110.99) (width 0.127) (layer "F.Cu") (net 2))
 (segment (start 132.7 110.99) (end 132.7 109.01) (width 0.127) (layer "F.Cu") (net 2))
 (segment (start 130.085 109.01) (end 132.7 109.01) (width 0.127) (layer "F.Cu") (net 2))
 (segment (start 158.7985 123.5585) (end 158.56 123.32) (width 0.127) (layer "F.Cu") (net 2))
 (segment (start 141.51 109.01) (end 141.3 108.8) (width 0.127) (layer "F.Cu") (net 2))
 (segment (start 106.1 109.3) (end 106.1 107.195) (width 0.127) (layer "F.Cu") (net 2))
 (via (at 126 108.9) (size 0.8) (drill 0.4) (layers "F.Cu" "B.Cu") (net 2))
 (via (at 107.6 108.5) (size 0.8) (drill 0.4) (layers "F.Cu" "B.Cu") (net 2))
 (via (at 139.9 109.9) (size 0.8) (drill 0.4) (layers "F.Cu" "B.Cu") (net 2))
 (via (at 133.6 109.9) (size 0.8) (drill 0.4) (layers "F.Cu" "B.Cu") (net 2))
 (segment (start 108.6635 109.5635) (end 119.7365 109.5635) (width 0.127) (layer "B.Cu") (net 2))
 (segment (start 107.6 108.5) (end 108.6635 109.5635) (width 0.127) (layer "B.Cu") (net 2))
 (segment (start 119.7365 109.5635) (end 121.0635 108.2365) (width 0.127) (layer "B.Cu") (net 2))
 (segment (start 126 108.9) (end 126.1 109) (width 0.127) (layer "B.Cu") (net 2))
 (segment (start 125.3365 108.2365) (end 126 108.9) (width 0.127) (layer "B.Cu") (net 2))
 (segment (start 133.6 109.9) (end 139.9 109.9) (width 0.127) (layer "B.Cu") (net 2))
 (segment (start 121.0635 108.2365) (end 125.3365 108.2365) (width 0.127) (layer "B.Cu") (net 2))
 (segment (start 131.155 107.245) (end 131.155 105) (width 0.127) (layer "F.Cu") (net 38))
 (segment (start 136.9 108.8) (end 136.9 106.6) (width 0.127) (layer "F.Cu") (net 38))
 (segment (start 136.9 108.8) (end 136.9 111.2) (width 0.127) (layer "F.Cu") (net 38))
 (segment (start 131.1 107.3) (end 131.155 107.245) (width 0.127) (layer "F.Cu") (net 38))
 (via (at 136.9 106.6) (size 0.8) (drill 0.4) (layers "F.Cu" "B.Cu") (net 38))
 (via (at 131.1 107.3) (size 0.8) (drill 0.4) (layers "F.Cu" "B.Cu") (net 38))
 (segment (start 136.9 106.6) (end 136.2365 107.2635) (width 0.127) (layer "B.Cu") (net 38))
 (segment (start 131.1365 107.2635) (end 131.1 107.3) (width 0.127) (layer "B.Cu") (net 38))
 (segment (start 136.2365 107.2635) (end 131.1365 107.2635) (width 0.127) (layer "B.Cu") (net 38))
 (segment (start 135.7 111.667) (end 136.6695 112.6365) (width 0.127) (layer "F.Cu") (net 32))
 (segment (start 138.5 112.6) (end 138.5365 112.6365) (width 0.127) (layer "F.Cu") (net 32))
 (segment (start 120.995 108.495) (end 120.995 105) (width 0.127) (layer "F.Cu") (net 32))
 (segment (start 121.4 108.9) (end 120.995 108.495) (width 0.127) (layer "F.Cu") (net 32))
 (segment (start 138.4635 112.6365) (end 138.5 112.6) (width 0.127) (layer "F.Cu") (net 32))
 (segment (start 138.5365 112.6365) (end 138.6 112.6365) (width 0.127) (layer "F.Cu") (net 32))
 (segment (start 136.6695 112.6365) (end 138.4635 112.6365) (width 0.127) (layer "F.Cu") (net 32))
 (segment (start 135.7 111.2) (end 135.7 111.667) (width 0.127) (layer "F.Cu") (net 32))
 (via (at 121.4 108.9) (size 0.8) (drill 0.4) (layers "F.Cu" "B.Cu") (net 32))
 (via (at 138.5 112.6) (size 0.8) (drill 0.4) (layers "F.Cu" "B.Cu") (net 32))
 (segment (start 121.4 108.9) (end 121.5 108.9) (width 0.127) (layer "B.Cu") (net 32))
 (segment (start 125.2 112.6) (end 121.4 108.9) (width 0.127) (layer "B.Cu") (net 32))
 (segment (start 138.5 112.6) (end 125.2 112.6) (width 0.127) (layer "B.Cu") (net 32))
 (segment (start 135.7 108.8) (end 135.7 106.6) (width 0.127) (layer "F.Cu") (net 33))
 (segment (start 118.455 108.755) (end 118.455 105) (width 0.127) (layer "F.Cu") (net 33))
 (segment (start 118.6 108.9) (end 118.455 108.755) (width 0.127) (layer "F.Cu") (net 33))
 (via (at 135.7 106.6) (size 0.8) (drill 0.4) (layers "F.Cu" "B.Cu") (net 33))
 (via (at 118.6 108.9) (size 0.8) (drill 0.4) (layers "F.Cu" "B.Cu") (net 33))
 (segment (start 118.6 108.7) (end 118.6 108.9) (width 0.127) (layer "B.Cu") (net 33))
 (segment (start 120.7 106.6) (end 118.6 108.7) (width 0.127) (layer "B.Cu") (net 33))
 (segment (start 118.6 108.9) (end 118.4 108.9) (width 0.127) (layer "B.Cu") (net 33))
 (segment (start 118.4 108.9) (end 118.4 108.9) (width 0.127) (layer "B.Cu") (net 33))
 (segment (start 135.7 106.6) (end 120.7 106.6) (width 0.127) (layer "B.Cu") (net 33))
 (segment (start 134.9 112.175948) (end 134.9 111.2) (width 0.127) (layer "F.Cu") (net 28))
 (segment (start 159.387 120.22) (end 158.56 120.22) (width 0.127) (layer "F.Cu") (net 28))
 (segment (start 158.56 119.22) (end 159.38 119.22) (width 0.127) (layer "F.Cu") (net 28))
 (segment (start 141.912026 119.187974) (end 134.9 112.175948) (width 0.127) (layer "F.Cu") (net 28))
 (segment (start 159.4735 120.1335) (end 159.387 120.22) (width 0.127) (layer "F.Cu") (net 28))
 (segment (start 141.944052 119.22) (end 141.912026 119.187974) (width 0.127) (layer "F.Cu") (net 28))
 (segment (start 158.56 119.22) (end 141.944052 119.22) (width 0.127) (layer "F.Cu") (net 28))
 (segment (start 159.4735 119.3135) (end 159.4735 120.1335) (width 0.127) (layer "F.Cu") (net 28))
 (segment (start 159.38 119.22) (end 159.4735 119.3135) (width 0.127) (layer "F.Cu") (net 28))
 (segment (start 157.6465 119.8065) (end 157.6465 120.6335) (width 0.127) (layer "F.Cu") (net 29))
 (segment (start 157.733 119.72) (end 157.6465 119.8065) (width 0.127) (layer "F.Cu") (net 29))
 (segment (start 157.5165 119.9365) (end 121.656773 119.9365) (width 0.127) (layer "F.Cu") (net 29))
 (segment (start 157.733 120.72) (end 158.56 120.72) (width 0.127) (layer "F.Cu") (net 29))
 (segment (start 157.6465 120.6335) (end 157.733 120.72) (width 0.127) (layer "F.Cu") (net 29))
 (segment (start 157.6465 119.8065) (end 157.5165 119.9365) (width 0.127) (layer "F.Cu") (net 29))
 (segment (start 134.9 106.518) (end 134.9 108.8) (width 0.127) (layer "F.Cu") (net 29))
 (segment (start 121.656773 119.9365) (end 117.9365 116.216227) (width 0.127) (layer "F.Cu") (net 29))
 (segment (start 117.9365 116.216227) (end 117.9 116.2) (width 0.127) (layer "F.Cu") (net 29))
 (segment (start 158.56 119.72) (end 157.733 119.72) (width 0.127) (layer "F.Cu") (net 29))
 (segment (start 132 103.4) (end 134.9 106.518) (width 0.127) (layer "F.Cu") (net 29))
 (segment (start 131.9415 103.5595) (end 132 103.4) (width 0.127) (layer "F.Cu") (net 29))
 (via (at 117.9 116.2) (size 0.8) (drill 0.4) (layers "F.Cu" "B.Cu") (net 29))
 (via (at 132 103.4) (size 0.8) (drill 0.4) (layers "F.Cu" "B.Cu") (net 29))
 (segment (start 106.9365 108.774831) (end 106.9365 108.225169) (width 0.127) (layer "B.Cu") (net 29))
 (segment (start 124.727 104.773273) (end 126.100273 103.4) (width 0.127) (layer "B.Cu") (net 29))
 (segment (start 106.9365 108.225169) (end 108.888669 106.273) (width 0.127) (layer "B.Cu") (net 29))
 (segment (start 124.727 106.273) (end 124.727 104.773273) (width 0.127) (layer "B.Cu") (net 29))
 (segment (start 126.100273 103.4) (end 132 103.4) (width 0.127) (layer "B.Cu") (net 29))
 (segment (start 114.361669 116.2) (end 106.9365 108.774831) (width 0.127) (layer "B.Cu") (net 29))
 (segment (start 108.888669 106.273) (end 124.727 106.273) (width 0.127) (layer "B.Cu") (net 29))
 (segment (start 117.9 116.2) (end 114.361669 116.2) (width 0.127) (layer "B.Cu") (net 29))
 (segment (start 158.56 117.72) (end 159.337 117.72) (width 0.127) (layer "F.Cu") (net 30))
 (segment (start 159.337 117.72) (end 159.387 117.77) (width 0.127) (layer "F.Cu") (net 30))
 (segment (start 158.56 117.42) (end 157.192 117.42) (width 0.127) (layer "F.Cu") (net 30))
 (segment (start 159.196314 122.52) (end 158.56 122.52) (width 0.127) (layer "F.Cu") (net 30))
 (segment (start 135.3 112.1135) (end 135.3 111.2) (width 0.127) (layer "F.Cu") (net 30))
 (segment (start 159.387 117.77) (end 160.303 117.77) (width 0.127) (layer "F.Cu") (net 30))
 (segment (start 138.1865 115) (end 135.3 112.1135) (width 0.127) (layer "F.Cu") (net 30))
 (segment (start 160.303 121.413314) (end 159.196314 122.52) (width 0.127) (layer "F.Cu") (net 30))
 (segment (start 158.56 117.42) (end 158.56 117.72) (width 0.127) (layer "F.Cu") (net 30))
 (segment (start 160.303 117.77) (end 160.303 121.413314) (width 0.127) (layer "F.Cu") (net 30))
 (segment (start 157.192 117.42) (end 154.642 114.87) (width 0.127) (layer "F.Cu") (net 30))
 (segment (start 158.56 122.22) (end 158.56 122.52) (width 0.127) (layer "F.Cu") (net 30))
 (segment (start 154.03 115.62) (end 156.63 118.22) (width 0.127) (layer "F.Cu") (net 1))
 (segment (start 156.63 118.22) (end 158.56 118.22) (width 0.127) (layer "F.Cu") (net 1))
 (segment (start 156.93 121.22) (end 154.03 124.12) (width 0.127) (layer "F.Cu") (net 25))
 (segment (start 158.56 121.22) (end 156.93 121.22) (width 0.127) (layer "F.Cu") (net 25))
 (segment (start 114.8015 106.1135) (end 113.6295 106.1135) (width 0.127) (layer "F.Cu") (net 9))
 (segment (start 113.6295 106.1135) (end 111.9 107.843) (width 0.127) (layer "F.Cu") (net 9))
 (segment (start 111.9 107.843) (end 111.9 108.8) (width 0.127) (layer "F.Cu") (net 9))
 (segment (start 115.915 105) (end 114.8015 106.1135) (width 0.127) (layer "F.Cu") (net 9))
 (segment (start 108.6815 110.9185) (end 106.9 109.137) (width 0.127) (layer "F.Cu") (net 8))
 (segment (start 108.961669 106.2) (end 112.175 106.2) (width 0.127) (layer "F.Cu") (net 8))
 (segment (start 111.8535 111.7135) (end 108.9865 111.7135) (width 0.127) (layer "F.Cu") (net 8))
 (segment (start 106.9 108.261669) (end 108.961669 106.2) (width 0.127) (layer "F.Cu") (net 8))
 (segment (start 108.6815 111.4085) (end 108.6815 110.9185) (width 0.127) (layer "F.Cu") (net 8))
 (segment (start 111.9 111.667) (end 111.8535 111.7135) (width 0.127) (layer "F.Cu") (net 8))
 (segment (start 108.9865 111.7135) (end 108.6815 111.4085) (width 0.127) (layer "F.Cu") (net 8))
 (segment (start 111.9 111.2) (end 111.9 111.667) (width 0.127) (layer "F.Cu") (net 8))
 (segment (start 106.9 109.137) (end 106.9 108.261669) (width 0.127) (layer "F.Cu") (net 8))
 (segment (start 112.175 106.2) (end 113.375 105) (width 0.127) (layer "F.Cu") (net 8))
 (segment (start 134.188948 112.0405) (end 134.5 111.729448) (width 0.127) (layer "F.Cu") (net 17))
 (segment (start 113.5 108.31) (end 113.5 107.843) (width 0.127) (layer "F.Cu") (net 17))
 (segment (start 120.7405 112.0405) (end 134.188948 112.0405) (width 0.127) (layer "F.Cu") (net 17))
 (segment (start 113.5465 107.7965) (end 117.107831 107.7965) (width 0.127) (layer "F.Cu") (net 17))
 (segment (start 117.107831 108.407831) (end 120.7405 112.0405) (width 0.127) (layer "F.Cu") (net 17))
 (segment (start 113.5 108.777) (end 113.5 108.31) (width 0.127) (layer "F.Cu") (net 17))
 (segment (start 117.107831 107.7965) (end 117.107831 108.407831) (width 0.127) (layer "F.Cu") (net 17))
 (segment (start 134.5 108.8) (end 134.5 111.2) (width 0.127) (layer "F.Cu") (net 17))
 (segment (start 134.5 111.729448) (end 134.5 111.2) (width 0.127) (layer "F.Cu") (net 17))
 (segment (start 113.5 107.843) (end 113.5465 107.7965) (width 0.127) (layer "F.Cu") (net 17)))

